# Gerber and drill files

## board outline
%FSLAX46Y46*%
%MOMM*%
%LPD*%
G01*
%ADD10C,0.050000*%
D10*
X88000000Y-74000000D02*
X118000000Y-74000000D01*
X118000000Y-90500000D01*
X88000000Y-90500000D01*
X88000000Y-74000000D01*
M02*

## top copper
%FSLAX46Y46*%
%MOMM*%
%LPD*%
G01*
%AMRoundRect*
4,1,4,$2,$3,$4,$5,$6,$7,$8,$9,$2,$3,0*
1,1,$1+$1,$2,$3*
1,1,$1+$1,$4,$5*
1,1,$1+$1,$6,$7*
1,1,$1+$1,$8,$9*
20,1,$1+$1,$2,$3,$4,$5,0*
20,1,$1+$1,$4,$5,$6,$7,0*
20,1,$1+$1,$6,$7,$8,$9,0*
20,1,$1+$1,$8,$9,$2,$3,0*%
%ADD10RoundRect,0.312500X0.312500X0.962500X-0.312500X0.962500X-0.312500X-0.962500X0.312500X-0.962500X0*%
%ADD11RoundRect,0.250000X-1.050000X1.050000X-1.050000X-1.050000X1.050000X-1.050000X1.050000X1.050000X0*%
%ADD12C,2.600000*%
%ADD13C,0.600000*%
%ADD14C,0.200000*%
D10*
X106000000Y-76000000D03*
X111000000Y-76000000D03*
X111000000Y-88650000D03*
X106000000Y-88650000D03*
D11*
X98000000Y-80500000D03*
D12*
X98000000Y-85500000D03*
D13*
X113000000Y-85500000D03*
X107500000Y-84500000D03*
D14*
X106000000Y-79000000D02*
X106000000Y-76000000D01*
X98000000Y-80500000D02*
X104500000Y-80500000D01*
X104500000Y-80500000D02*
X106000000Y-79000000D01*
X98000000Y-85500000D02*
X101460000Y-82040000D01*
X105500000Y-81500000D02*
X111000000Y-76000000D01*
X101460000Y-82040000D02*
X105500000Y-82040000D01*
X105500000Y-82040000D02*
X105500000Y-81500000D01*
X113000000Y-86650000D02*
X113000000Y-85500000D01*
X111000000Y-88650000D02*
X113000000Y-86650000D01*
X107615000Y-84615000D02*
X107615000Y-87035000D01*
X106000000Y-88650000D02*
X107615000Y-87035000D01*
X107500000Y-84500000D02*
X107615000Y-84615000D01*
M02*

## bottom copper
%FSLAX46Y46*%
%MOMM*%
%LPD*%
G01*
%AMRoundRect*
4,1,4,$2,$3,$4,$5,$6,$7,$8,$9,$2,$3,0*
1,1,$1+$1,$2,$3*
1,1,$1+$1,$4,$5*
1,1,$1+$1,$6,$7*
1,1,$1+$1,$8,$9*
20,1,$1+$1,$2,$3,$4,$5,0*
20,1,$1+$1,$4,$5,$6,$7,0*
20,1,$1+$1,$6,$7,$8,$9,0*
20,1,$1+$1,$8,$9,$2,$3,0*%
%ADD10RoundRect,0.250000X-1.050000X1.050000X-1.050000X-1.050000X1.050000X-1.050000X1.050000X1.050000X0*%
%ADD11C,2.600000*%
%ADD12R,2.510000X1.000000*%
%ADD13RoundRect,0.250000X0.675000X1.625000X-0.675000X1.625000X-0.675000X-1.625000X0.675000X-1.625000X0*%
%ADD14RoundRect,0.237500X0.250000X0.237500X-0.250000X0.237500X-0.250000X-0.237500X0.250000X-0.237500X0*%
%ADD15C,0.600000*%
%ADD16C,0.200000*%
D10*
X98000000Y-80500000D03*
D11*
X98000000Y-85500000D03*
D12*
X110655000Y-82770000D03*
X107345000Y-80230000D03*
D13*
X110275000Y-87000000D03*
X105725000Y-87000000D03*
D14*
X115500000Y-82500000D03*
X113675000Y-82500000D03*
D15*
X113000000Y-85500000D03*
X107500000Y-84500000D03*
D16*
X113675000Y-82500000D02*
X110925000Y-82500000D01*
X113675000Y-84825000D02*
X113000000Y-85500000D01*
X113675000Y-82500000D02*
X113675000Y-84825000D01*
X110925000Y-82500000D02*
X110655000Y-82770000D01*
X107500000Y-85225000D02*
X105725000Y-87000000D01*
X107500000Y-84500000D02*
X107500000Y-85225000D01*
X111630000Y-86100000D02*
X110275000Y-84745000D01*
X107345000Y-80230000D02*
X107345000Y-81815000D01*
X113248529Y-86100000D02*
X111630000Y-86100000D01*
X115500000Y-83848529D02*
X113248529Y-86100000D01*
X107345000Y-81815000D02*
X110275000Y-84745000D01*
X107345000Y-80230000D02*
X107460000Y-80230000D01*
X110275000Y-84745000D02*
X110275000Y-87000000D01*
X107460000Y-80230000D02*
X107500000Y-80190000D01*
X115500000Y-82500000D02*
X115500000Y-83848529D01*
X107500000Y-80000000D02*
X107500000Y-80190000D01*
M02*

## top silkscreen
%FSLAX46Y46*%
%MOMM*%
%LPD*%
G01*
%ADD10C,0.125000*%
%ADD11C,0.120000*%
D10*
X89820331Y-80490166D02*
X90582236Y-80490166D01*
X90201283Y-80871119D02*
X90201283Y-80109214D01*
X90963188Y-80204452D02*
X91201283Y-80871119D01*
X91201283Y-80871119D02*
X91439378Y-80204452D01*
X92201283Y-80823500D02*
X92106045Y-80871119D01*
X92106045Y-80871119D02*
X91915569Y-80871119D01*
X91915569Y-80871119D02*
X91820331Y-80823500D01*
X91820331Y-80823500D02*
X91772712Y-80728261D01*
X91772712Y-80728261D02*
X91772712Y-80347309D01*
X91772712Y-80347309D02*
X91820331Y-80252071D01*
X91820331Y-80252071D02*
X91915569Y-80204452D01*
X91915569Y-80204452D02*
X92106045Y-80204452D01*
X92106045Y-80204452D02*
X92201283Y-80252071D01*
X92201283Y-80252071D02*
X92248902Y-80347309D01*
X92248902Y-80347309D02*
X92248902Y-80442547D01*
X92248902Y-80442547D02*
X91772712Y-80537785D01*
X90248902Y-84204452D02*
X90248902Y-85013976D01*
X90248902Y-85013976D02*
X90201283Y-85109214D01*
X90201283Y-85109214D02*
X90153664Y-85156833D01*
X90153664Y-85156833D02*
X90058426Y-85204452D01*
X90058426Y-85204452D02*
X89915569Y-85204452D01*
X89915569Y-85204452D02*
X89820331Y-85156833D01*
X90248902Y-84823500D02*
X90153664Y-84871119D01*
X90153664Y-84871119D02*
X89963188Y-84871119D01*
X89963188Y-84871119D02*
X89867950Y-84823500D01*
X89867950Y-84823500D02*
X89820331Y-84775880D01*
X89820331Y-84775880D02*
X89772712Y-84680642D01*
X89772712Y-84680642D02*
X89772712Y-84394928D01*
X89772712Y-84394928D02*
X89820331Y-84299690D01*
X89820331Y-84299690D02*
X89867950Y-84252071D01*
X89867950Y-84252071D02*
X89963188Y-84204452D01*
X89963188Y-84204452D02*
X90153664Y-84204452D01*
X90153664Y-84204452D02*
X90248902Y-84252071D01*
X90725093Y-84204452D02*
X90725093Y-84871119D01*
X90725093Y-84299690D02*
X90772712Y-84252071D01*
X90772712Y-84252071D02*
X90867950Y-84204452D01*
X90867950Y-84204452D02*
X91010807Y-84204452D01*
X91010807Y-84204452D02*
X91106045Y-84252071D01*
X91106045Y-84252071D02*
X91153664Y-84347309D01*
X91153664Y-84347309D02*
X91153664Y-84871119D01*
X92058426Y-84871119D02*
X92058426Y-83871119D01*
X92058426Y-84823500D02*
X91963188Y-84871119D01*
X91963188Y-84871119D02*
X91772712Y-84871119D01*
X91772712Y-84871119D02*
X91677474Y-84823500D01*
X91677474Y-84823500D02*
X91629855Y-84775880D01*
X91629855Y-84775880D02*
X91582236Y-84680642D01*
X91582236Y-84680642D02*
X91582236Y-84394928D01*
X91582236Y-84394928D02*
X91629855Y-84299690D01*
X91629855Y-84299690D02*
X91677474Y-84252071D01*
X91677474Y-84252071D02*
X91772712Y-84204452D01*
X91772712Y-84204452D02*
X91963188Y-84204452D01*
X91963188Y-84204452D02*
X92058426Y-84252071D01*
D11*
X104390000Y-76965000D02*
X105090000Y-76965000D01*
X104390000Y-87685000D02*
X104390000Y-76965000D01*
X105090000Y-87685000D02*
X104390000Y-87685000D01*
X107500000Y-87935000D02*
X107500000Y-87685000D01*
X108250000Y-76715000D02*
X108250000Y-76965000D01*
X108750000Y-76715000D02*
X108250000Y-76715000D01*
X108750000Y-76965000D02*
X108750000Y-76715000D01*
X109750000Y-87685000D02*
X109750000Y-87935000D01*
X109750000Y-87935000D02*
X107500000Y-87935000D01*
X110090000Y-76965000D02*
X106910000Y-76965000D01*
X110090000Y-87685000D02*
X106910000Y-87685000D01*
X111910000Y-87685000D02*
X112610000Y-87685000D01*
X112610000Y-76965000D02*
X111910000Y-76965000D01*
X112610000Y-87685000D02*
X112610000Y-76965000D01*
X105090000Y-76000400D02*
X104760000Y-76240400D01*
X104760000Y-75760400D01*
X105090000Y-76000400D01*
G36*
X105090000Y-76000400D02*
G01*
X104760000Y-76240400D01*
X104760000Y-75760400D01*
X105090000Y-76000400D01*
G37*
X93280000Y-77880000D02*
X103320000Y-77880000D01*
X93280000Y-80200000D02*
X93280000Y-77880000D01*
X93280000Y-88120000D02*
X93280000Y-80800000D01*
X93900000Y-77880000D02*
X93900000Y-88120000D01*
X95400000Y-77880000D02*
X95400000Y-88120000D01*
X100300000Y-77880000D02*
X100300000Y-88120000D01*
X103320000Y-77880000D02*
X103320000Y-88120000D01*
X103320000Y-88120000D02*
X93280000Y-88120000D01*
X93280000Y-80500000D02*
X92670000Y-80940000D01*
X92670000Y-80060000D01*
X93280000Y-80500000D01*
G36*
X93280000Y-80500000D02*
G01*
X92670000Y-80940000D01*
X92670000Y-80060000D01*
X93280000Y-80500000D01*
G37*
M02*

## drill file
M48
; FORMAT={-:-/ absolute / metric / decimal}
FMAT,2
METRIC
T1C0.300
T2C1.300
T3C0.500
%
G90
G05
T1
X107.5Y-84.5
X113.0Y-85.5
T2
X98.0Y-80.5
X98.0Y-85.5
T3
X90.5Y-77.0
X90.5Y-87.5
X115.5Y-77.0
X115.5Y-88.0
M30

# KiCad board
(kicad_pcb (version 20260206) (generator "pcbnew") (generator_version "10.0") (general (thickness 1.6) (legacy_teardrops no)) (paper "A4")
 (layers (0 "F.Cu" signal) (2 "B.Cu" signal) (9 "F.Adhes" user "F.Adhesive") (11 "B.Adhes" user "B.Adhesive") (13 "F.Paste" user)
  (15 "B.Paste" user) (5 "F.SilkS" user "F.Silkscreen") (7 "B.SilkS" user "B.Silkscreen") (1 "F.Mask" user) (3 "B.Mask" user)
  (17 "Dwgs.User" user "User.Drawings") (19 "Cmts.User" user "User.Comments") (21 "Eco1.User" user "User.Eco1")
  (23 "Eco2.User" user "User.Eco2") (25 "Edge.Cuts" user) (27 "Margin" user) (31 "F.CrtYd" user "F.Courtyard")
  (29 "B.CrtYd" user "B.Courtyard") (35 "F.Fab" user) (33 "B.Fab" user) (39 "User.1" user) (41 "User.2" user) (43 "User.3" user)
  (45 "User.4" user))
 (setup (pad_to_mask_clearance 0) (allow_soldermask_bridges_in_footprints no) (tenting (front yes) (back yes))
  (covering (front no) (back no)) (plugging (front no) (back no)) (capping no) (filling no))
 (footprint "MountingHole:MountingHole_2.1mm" (layer "F.Cu") (at 90.5 87.5)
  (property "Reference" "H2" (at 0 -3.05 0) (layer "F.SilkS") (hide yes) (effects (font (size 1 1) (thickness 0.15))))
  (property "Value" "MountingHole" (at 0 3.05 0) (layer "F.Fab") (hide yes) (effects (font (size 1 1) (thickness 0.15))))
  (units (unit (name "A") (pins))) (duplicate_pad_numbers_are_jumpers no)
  (pad "" np_thru_hole circle (at 0 0) (size 0.5 0.5) (drill 0.5) (layers "*.Cu" "*.Mask")))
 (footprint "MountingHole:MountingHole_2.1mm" (layer "F.Cu") (at 115.5 77)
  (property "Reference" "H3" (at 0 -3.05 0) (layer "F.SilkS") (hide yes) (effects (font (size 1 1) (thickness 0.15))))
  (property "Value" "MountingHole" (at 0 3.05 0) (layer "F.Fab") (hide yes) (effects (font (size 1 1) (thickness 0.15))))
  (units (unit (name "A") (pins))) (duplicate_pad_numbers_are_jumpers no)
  (pad "" np_thru_hole circle (at 0 0) (size 0.5 0.5) (drill 0.5) (layers "*.Cu" "*.Mask")))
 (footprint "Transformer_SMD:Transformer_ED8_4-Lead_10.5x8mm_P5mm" (layer "F.Cu") (at 108.5 82.325)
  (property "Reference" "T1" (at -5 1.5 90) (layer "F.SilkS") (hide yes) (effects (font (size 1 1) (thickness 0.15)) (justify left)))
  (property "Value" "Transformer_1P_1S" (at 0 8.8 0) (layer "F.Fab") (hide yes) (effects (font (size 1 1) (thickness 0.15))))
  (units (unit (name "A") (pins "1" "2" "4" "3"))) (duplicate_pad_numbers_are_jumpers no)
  (fp_line (start -4.11 -5.36) (end -3.41 -5.36) (stroke (width 0.12) (type default)) (layer "F.SilkS"))
  (fp_line (start -4.11 5.36) (end -4.11 -5.36) (stroke (width 0.12) (type default)) (layer "F.SilkS"))
  (fp_line (start -3.41 5.36) (end -4.11 5.36) (stroke (width 0.12) (type default)) (layer "F.SilkS"))
  (fp_line (start -1 5.61) (end -1 5.36) (stroke (width 0.12) (type default)) (layer "F.SilkS"))
  (fp_line (start -0.25 -5.61) (end -0.25 -5.36) (stroke (width 0.12) (type default)) (layer "F.SilkS"))
  (fp_line (start 0.25 -5.61) (end -0.25 -5.61) (stroke (width 0.12) (type default)) (layer "F.SilkS"))
  (fp_line (start 0.25 -5.36) (end 0.25 -5.61) (stroke (width 0.12) (type default)) (layer "F.SilkS"))
  (fp_line (start 1.25 5.36) (end 1.25 5.61) (stroke (width 0.12) (type default)) (layer "F.SilkS"))
  (fp_line (start 1.25 5.61) (end -1 5.61) (stroke (width 0.12) (type default)) (layer "F.SilkS"))
  (fp_line (start 1.59 -5.36) (end -1.59 -5.36) (stroke (width 0.12) (type default)) (layer "F.SilkS"))
  (fp_line (start 1.59 5.36) (end -1.59 5.36) (stroke (width 0.12) (type default)) (layer "F.SilkS"))
  (fp_line (start 3.41 5.36) (end 4.11 5.36) (stroke (width 0.12) (type default)) (layer "F.SilkS"))
  (fp_line (start 4.11 -5.36) (end 3.41 -5.36) (stroke (width 0.12) (type default)) (layer "F.SilkS"))
  (fp_line (start 4.11 5.36) (end 4.11 -5.36) (stroke (width 0.12) (type default)) (layer "F.SilkS"))
  (fp_poly
   (pts (xy -3.41 -6.3246) (xy -3.74 -6.0846) (xy -3.74 -6.5646) (xy -3.41 -6.3246)) (stroke (width 0.12) (type solid)) (fill yes)
   (layer "F.SilkS"))
  (pad "1" smd roundrect (at -2.5 -6.325 180) (size 1.25 2.55) (layers "F.Cu" "F.Mask" "F.Paste") (roundrect_rratio 0.25)
   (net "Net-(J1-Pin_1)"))
  (pad "2" smd roundrect (at 2.5 -6.325 180) (size 1.25 2.55) (layers "F.Cu" "F.Mask" "F.Paste") (roundrect_rratio 0.25)
   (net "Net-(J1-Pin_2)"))
  (pad "3" smd roundrect (at 2.5 6.325 180) (size 1.25 2.55) (layers "F.Cu" "F.Mask" "F.Paste") (roundrect_rratio 0.25)
   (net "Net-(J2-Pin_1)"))
  (pad "4" smd roundrect (at -2.5 6.325 180) (size 1.25 2.55) (layers "F.Cu" "F.Mask" "F.Paste") (roundrect_rratio 0.25) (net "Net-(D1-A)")))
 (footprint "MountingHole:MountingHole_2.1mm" (layer "F.Cu") (at 90.5 77)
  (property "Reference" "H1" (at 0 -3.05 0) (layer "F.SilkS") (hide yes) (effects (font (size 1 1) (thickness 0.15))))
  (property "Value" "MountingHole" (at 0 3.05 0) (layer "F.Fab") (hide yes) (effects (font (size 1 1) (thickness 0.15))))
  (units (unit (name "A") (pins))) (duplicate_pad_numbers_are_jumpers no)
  (pad "" np_thru_hole circle (at 0 0) (size 0.5 0.5) (drill 0.5) (layers "*.Cu" "*.Mask")))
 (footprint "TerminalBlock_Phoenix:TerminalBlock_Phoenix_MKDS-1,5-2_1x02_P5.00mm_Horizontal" (layer "F.Cu") (at 98 80.5 -90)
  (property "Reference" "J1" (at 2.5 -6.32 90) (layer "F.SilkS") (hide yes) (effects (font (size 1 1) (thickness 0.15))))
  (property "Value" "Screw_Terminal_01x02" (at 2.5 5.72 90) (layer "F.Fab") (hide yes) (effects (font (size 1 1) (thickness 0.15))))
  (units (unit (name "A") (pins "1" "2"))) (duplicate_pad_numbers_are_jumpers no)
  (fp_line (start -2.62 4.72) (end -2.62 -5.32) (stroke (width 0.12) (type solid)) (layer "F.SilkS"))
  (fp_line (start -0.3 4.72) (end -2.62 4.72) (stroke (width 0.12) (type solid)) (layer "F.SilkS"))
  (fp_line (start 7.62 4.72) (end 0.3 4.72) (stroke (width 0.12) (type solid)) (layer "F.SilkS"))
  (fp_line (start -2.62 4.1) (end 7.62 4.1) (stroke (width 0.12) (type solid)) (layer "F.SilkS"))
  (fp_line (start -2.62 2.6) (end 7.62 2.6) (stroke (width 0.12) (type solid)) (layer "F.SilkS"))
  (fp_line (start -2.62 -2.3) (end 7.62 -2.3) (stroke (width 0.12) (type solid)) (layer "F.SilkS"))
  (fp_line (start -2.62 -5.32) (end 7.62 -5.32) (stroke (width 0.12) (type solid)) (layer "F.SilkS"))
  (fp_line (start 7.62 -5.32) (end 7.62 4.72) (stroke (width 0.12) (type solid)) (layer "F.SilkS"))
  (fp_poly (pts (xy 0 4.72) (xy 0.44 5.33) (xy -0.44 5.33)) (stroke (width 0.12) (type solid)) (fill yes) (layer "F.SilkS"))
  (pad "1" thru_hole roundrect (at 0 0 270) (size 2.6 2.6) (drill 1.3) (layers "*.Cu" "*.Mask") (remove_unused_layers no)
   (roundrect_rratio 0.096154) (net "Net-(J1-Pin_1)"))
  (pad "2" thru_hole circle (at 5 0 270) (size 2.6 2.6) (drill 1.3) (layers "*.Cu" "*.Mask") (remove_unused_layers no)
   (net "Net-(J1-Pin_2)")))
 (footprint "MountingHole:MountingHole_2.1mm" (layer "F.Cu") (at 115.5 88)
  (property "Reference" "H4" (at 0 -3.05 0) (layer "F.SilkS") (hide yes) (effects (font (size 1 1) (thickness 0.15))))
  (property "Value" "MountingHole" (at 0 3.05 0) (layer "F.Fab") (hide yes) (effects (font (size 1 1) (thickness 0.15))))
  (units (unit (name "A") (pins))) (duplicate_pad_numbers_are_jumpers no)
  (pad "" np_thru_hole circle (at 0 0) (size 0.5 0.5) (drill 0.5) (layers "*.Cu" "*.Mask")))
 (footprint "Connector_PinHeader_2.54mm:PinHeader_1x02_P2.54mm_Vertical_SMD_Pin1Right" (layer "B.Cu") (at 109 81.5)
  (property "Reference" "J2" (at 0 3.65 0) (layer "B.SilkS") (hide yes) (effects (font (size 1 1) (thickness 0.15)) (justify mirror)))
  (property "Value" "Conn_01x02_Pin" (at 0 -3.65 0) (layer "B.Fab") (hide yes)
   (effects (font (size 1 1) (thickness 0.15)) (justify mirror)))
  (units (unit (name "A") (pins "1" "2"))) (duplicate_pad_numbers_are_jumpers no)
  (pad "1" smd rect (at 1.655 1.27) (size 2.51 1) (layers "B.Cu" "B.Mask" "B.Paste") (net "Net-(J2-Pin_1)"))
  (pad "2" smd rect (at -1.655 -1.27) (size 2.51 1) (layers "B.Cu" "B.Mask" "B.Paste") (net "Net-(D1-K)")))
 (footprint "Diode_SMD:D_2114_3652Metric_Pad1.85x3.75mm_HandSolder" (layer "B.Cu") (at 108 87 180)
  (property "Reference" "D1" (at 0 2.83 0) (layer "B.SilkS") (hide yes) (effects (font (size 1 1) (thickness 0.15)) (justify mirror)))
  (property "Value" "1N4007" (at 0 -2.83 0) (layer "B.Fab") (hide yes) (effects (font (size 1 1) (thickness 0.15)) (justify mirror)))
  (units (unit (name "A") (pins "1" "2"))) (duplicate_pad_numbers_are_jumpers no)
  (pad "1" smd roundrect (at -2.275 0 180) (size 1.85 3.75) (layers "B.Cu" "B.Mask" "B.Paste") (roundrect_rratio 0.135135)
   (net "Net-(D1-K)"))
  (pad "2" smd roundrect (at 2.275 0 180) (size 1.85 3.75) (layers "B.Cu" "B.Mask" "B.Paste") (roundrect_rratio 0.135135) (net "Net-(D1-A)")))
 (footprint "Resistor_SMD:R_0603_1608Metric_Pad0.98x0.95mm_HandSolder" (layer "B.Cu") (at 114.5875 82.5 180)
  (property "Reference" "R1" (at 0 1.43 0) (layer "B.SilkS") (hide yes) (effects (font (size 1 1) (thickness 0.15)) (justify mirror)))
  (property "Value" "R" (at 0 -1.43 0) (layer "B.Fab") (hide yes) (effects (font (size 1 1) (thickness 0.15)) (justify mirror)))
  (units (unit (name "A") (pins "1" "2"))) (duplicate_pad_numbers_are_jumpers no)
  (pad "1" smd roundrect (at -0.9125 0 180) (size 0.975 0.95) (layers "B.Cu" "B.Mask" "B.Paste") (roundrect_rratio 0.25) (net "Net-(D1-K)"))
  (pad "2" smd roundrect (at 0.9125 0 180) (size 0.975 0.95) (layers "B.Cu" "B.Mask" "B.Paste") (roundrect_rratio 0.25)
   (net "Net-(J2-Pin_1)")))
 (gr_rect (start 88 74) (end 118 90.5) (stroke (width 0.05) (type default)) (fill no) (layer "Edge.Cuts"))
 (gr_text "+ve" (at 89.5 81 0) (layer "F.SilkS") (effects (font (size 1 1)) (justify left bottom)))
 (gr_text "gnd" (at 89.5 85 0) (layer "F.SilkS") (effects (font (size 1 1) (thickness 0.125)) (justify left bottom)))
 (segment (start 106 79) (end 106 76) (width 0.2) (layer "F.Cu") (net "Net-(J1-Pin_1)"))
 (segment (start 98 80.5) (end 104.5 80.5) (width 0.2) (layer "F.Cu") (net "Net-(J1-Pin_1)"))
 (segment (start 104.5 80.5) (end 106 79) (width 0.2) (layer "F.Cu") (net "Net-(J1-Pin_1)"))
 (segment (start 98 85.5) (end 101.46 82.04) (width 0.2) (layer "F.Cu") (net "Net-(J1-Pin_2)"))
 (segment (start 105.5 81.5) (end 111 76) (width 0.2) (layer "F.Cu") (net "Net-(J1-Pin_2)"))
 (segment (start 101.46 82.04) (end 105.5 82.04) (width 0.2) (layer "F.Cu") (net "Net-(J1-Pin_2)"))
 (segment (start 105.5 82.04) (end 105.5 81.5) (width 0.2) (layer "F.Cu") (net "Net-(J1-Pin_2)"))
 (segment (start 113 86.65) (end 113 85.5) (width 0.2) (layer "F.Cu") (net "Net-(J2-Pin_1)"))
 (segment (start 111 88.65) (end 113 86.65) (width 0.2) (layer "F.Cu") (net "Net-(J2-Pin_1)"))
 (via (at 113 85.5) (size 0.6) (drill 0.3) (layers "F.Cu" "B.Cu") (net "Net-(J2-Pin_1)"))
 (segment (start 113.675 82.5) (end 110.925 82.5) (width 0.2) (layer "B.Cu") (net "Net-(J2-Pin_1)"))
 (segment (start 113.675 84.825) (end 113 85.5) (width 0.2) (layer "B.Cu") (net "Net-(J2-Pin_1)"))
 (segment (start 113.675 82.5) (end 113.675 84.825) (width 0.2) (layer "B.Cu") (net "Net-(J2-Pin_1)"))
 (segment (start 110.925 82.5) (end 110.655 82.77) (width 0.2) (layer "B.Cu") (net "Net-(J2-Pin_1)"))
 (segment (start 107.615 84.615) (end 107.615 87.035) (width 0.2) (layer "F.Cu") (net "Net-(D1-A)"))
 (segment (start 106 88.65) (end 107.615 87.035) (width 0.2) (layer "F.Cu") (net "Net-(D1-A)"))
 (segment (start 107.5 84.5) (end 107.615 84.615) (width 0.2) (layer "F.Cu") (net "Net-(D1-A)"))
 (via (at 107.5 84.5) (size 0.6) (drill 0.3) (layers "F.Cu" "B.Cu") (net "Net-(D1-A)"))
 (segment (start 107.5 85.225) (end 105.725 87) (width 0.2) (layer "B.Cu") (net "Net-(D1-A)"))
 (segment (start 107.5 84.5) (end 107.5 85.225) (width 0.2) (layer "B.Cu") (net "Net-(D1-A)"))
 (segment (start 111.63 86.1) (end 110.275 84.745) (width 0.2) (layer "B.Cu") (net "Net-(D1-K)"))
 (segment (start 107.345 80.23) (end 107.345 81.815) (width 0.2) (layer "B.Cu") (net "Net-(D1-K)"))
 (segment (start 113.248529 86.1) (end 111.63 86.1) (width 0.2) (layer "B.Cu") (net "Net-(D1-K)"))
 (segment (start 115.5 83.848529) (end 113.248529 86.1) (width 0.2) (layer "B.Cu") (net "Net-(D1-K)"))
 (segment (start 107.345 81.815) (end 110.275 84.745) (width 0.2) (layer "B.Cu") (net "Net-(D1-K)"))
 (segment (start 107.345 80.23) (end 107.46 80.23) (width 0.2) (layer "B.Cu") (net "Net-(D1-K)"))
 (segment (start 110.275 84.745) (end 110.275 87) (width 0.2) (layer "B.Cu") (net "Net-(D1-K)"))
 (segment (start 107.46 80.23) (end 107.5 80.19) (width 0.2) (layer "B.Cu") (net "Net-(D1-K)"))
 (segment (start 115.5 82.5) (end 115.5 83.848529) (width 0.2) (layer "B.Cu") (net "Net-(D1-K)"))
 (segment (start 107.5 80) (end 107.5 80.19) (width 0.2) (layer "B.Cu") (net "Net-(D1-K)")))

